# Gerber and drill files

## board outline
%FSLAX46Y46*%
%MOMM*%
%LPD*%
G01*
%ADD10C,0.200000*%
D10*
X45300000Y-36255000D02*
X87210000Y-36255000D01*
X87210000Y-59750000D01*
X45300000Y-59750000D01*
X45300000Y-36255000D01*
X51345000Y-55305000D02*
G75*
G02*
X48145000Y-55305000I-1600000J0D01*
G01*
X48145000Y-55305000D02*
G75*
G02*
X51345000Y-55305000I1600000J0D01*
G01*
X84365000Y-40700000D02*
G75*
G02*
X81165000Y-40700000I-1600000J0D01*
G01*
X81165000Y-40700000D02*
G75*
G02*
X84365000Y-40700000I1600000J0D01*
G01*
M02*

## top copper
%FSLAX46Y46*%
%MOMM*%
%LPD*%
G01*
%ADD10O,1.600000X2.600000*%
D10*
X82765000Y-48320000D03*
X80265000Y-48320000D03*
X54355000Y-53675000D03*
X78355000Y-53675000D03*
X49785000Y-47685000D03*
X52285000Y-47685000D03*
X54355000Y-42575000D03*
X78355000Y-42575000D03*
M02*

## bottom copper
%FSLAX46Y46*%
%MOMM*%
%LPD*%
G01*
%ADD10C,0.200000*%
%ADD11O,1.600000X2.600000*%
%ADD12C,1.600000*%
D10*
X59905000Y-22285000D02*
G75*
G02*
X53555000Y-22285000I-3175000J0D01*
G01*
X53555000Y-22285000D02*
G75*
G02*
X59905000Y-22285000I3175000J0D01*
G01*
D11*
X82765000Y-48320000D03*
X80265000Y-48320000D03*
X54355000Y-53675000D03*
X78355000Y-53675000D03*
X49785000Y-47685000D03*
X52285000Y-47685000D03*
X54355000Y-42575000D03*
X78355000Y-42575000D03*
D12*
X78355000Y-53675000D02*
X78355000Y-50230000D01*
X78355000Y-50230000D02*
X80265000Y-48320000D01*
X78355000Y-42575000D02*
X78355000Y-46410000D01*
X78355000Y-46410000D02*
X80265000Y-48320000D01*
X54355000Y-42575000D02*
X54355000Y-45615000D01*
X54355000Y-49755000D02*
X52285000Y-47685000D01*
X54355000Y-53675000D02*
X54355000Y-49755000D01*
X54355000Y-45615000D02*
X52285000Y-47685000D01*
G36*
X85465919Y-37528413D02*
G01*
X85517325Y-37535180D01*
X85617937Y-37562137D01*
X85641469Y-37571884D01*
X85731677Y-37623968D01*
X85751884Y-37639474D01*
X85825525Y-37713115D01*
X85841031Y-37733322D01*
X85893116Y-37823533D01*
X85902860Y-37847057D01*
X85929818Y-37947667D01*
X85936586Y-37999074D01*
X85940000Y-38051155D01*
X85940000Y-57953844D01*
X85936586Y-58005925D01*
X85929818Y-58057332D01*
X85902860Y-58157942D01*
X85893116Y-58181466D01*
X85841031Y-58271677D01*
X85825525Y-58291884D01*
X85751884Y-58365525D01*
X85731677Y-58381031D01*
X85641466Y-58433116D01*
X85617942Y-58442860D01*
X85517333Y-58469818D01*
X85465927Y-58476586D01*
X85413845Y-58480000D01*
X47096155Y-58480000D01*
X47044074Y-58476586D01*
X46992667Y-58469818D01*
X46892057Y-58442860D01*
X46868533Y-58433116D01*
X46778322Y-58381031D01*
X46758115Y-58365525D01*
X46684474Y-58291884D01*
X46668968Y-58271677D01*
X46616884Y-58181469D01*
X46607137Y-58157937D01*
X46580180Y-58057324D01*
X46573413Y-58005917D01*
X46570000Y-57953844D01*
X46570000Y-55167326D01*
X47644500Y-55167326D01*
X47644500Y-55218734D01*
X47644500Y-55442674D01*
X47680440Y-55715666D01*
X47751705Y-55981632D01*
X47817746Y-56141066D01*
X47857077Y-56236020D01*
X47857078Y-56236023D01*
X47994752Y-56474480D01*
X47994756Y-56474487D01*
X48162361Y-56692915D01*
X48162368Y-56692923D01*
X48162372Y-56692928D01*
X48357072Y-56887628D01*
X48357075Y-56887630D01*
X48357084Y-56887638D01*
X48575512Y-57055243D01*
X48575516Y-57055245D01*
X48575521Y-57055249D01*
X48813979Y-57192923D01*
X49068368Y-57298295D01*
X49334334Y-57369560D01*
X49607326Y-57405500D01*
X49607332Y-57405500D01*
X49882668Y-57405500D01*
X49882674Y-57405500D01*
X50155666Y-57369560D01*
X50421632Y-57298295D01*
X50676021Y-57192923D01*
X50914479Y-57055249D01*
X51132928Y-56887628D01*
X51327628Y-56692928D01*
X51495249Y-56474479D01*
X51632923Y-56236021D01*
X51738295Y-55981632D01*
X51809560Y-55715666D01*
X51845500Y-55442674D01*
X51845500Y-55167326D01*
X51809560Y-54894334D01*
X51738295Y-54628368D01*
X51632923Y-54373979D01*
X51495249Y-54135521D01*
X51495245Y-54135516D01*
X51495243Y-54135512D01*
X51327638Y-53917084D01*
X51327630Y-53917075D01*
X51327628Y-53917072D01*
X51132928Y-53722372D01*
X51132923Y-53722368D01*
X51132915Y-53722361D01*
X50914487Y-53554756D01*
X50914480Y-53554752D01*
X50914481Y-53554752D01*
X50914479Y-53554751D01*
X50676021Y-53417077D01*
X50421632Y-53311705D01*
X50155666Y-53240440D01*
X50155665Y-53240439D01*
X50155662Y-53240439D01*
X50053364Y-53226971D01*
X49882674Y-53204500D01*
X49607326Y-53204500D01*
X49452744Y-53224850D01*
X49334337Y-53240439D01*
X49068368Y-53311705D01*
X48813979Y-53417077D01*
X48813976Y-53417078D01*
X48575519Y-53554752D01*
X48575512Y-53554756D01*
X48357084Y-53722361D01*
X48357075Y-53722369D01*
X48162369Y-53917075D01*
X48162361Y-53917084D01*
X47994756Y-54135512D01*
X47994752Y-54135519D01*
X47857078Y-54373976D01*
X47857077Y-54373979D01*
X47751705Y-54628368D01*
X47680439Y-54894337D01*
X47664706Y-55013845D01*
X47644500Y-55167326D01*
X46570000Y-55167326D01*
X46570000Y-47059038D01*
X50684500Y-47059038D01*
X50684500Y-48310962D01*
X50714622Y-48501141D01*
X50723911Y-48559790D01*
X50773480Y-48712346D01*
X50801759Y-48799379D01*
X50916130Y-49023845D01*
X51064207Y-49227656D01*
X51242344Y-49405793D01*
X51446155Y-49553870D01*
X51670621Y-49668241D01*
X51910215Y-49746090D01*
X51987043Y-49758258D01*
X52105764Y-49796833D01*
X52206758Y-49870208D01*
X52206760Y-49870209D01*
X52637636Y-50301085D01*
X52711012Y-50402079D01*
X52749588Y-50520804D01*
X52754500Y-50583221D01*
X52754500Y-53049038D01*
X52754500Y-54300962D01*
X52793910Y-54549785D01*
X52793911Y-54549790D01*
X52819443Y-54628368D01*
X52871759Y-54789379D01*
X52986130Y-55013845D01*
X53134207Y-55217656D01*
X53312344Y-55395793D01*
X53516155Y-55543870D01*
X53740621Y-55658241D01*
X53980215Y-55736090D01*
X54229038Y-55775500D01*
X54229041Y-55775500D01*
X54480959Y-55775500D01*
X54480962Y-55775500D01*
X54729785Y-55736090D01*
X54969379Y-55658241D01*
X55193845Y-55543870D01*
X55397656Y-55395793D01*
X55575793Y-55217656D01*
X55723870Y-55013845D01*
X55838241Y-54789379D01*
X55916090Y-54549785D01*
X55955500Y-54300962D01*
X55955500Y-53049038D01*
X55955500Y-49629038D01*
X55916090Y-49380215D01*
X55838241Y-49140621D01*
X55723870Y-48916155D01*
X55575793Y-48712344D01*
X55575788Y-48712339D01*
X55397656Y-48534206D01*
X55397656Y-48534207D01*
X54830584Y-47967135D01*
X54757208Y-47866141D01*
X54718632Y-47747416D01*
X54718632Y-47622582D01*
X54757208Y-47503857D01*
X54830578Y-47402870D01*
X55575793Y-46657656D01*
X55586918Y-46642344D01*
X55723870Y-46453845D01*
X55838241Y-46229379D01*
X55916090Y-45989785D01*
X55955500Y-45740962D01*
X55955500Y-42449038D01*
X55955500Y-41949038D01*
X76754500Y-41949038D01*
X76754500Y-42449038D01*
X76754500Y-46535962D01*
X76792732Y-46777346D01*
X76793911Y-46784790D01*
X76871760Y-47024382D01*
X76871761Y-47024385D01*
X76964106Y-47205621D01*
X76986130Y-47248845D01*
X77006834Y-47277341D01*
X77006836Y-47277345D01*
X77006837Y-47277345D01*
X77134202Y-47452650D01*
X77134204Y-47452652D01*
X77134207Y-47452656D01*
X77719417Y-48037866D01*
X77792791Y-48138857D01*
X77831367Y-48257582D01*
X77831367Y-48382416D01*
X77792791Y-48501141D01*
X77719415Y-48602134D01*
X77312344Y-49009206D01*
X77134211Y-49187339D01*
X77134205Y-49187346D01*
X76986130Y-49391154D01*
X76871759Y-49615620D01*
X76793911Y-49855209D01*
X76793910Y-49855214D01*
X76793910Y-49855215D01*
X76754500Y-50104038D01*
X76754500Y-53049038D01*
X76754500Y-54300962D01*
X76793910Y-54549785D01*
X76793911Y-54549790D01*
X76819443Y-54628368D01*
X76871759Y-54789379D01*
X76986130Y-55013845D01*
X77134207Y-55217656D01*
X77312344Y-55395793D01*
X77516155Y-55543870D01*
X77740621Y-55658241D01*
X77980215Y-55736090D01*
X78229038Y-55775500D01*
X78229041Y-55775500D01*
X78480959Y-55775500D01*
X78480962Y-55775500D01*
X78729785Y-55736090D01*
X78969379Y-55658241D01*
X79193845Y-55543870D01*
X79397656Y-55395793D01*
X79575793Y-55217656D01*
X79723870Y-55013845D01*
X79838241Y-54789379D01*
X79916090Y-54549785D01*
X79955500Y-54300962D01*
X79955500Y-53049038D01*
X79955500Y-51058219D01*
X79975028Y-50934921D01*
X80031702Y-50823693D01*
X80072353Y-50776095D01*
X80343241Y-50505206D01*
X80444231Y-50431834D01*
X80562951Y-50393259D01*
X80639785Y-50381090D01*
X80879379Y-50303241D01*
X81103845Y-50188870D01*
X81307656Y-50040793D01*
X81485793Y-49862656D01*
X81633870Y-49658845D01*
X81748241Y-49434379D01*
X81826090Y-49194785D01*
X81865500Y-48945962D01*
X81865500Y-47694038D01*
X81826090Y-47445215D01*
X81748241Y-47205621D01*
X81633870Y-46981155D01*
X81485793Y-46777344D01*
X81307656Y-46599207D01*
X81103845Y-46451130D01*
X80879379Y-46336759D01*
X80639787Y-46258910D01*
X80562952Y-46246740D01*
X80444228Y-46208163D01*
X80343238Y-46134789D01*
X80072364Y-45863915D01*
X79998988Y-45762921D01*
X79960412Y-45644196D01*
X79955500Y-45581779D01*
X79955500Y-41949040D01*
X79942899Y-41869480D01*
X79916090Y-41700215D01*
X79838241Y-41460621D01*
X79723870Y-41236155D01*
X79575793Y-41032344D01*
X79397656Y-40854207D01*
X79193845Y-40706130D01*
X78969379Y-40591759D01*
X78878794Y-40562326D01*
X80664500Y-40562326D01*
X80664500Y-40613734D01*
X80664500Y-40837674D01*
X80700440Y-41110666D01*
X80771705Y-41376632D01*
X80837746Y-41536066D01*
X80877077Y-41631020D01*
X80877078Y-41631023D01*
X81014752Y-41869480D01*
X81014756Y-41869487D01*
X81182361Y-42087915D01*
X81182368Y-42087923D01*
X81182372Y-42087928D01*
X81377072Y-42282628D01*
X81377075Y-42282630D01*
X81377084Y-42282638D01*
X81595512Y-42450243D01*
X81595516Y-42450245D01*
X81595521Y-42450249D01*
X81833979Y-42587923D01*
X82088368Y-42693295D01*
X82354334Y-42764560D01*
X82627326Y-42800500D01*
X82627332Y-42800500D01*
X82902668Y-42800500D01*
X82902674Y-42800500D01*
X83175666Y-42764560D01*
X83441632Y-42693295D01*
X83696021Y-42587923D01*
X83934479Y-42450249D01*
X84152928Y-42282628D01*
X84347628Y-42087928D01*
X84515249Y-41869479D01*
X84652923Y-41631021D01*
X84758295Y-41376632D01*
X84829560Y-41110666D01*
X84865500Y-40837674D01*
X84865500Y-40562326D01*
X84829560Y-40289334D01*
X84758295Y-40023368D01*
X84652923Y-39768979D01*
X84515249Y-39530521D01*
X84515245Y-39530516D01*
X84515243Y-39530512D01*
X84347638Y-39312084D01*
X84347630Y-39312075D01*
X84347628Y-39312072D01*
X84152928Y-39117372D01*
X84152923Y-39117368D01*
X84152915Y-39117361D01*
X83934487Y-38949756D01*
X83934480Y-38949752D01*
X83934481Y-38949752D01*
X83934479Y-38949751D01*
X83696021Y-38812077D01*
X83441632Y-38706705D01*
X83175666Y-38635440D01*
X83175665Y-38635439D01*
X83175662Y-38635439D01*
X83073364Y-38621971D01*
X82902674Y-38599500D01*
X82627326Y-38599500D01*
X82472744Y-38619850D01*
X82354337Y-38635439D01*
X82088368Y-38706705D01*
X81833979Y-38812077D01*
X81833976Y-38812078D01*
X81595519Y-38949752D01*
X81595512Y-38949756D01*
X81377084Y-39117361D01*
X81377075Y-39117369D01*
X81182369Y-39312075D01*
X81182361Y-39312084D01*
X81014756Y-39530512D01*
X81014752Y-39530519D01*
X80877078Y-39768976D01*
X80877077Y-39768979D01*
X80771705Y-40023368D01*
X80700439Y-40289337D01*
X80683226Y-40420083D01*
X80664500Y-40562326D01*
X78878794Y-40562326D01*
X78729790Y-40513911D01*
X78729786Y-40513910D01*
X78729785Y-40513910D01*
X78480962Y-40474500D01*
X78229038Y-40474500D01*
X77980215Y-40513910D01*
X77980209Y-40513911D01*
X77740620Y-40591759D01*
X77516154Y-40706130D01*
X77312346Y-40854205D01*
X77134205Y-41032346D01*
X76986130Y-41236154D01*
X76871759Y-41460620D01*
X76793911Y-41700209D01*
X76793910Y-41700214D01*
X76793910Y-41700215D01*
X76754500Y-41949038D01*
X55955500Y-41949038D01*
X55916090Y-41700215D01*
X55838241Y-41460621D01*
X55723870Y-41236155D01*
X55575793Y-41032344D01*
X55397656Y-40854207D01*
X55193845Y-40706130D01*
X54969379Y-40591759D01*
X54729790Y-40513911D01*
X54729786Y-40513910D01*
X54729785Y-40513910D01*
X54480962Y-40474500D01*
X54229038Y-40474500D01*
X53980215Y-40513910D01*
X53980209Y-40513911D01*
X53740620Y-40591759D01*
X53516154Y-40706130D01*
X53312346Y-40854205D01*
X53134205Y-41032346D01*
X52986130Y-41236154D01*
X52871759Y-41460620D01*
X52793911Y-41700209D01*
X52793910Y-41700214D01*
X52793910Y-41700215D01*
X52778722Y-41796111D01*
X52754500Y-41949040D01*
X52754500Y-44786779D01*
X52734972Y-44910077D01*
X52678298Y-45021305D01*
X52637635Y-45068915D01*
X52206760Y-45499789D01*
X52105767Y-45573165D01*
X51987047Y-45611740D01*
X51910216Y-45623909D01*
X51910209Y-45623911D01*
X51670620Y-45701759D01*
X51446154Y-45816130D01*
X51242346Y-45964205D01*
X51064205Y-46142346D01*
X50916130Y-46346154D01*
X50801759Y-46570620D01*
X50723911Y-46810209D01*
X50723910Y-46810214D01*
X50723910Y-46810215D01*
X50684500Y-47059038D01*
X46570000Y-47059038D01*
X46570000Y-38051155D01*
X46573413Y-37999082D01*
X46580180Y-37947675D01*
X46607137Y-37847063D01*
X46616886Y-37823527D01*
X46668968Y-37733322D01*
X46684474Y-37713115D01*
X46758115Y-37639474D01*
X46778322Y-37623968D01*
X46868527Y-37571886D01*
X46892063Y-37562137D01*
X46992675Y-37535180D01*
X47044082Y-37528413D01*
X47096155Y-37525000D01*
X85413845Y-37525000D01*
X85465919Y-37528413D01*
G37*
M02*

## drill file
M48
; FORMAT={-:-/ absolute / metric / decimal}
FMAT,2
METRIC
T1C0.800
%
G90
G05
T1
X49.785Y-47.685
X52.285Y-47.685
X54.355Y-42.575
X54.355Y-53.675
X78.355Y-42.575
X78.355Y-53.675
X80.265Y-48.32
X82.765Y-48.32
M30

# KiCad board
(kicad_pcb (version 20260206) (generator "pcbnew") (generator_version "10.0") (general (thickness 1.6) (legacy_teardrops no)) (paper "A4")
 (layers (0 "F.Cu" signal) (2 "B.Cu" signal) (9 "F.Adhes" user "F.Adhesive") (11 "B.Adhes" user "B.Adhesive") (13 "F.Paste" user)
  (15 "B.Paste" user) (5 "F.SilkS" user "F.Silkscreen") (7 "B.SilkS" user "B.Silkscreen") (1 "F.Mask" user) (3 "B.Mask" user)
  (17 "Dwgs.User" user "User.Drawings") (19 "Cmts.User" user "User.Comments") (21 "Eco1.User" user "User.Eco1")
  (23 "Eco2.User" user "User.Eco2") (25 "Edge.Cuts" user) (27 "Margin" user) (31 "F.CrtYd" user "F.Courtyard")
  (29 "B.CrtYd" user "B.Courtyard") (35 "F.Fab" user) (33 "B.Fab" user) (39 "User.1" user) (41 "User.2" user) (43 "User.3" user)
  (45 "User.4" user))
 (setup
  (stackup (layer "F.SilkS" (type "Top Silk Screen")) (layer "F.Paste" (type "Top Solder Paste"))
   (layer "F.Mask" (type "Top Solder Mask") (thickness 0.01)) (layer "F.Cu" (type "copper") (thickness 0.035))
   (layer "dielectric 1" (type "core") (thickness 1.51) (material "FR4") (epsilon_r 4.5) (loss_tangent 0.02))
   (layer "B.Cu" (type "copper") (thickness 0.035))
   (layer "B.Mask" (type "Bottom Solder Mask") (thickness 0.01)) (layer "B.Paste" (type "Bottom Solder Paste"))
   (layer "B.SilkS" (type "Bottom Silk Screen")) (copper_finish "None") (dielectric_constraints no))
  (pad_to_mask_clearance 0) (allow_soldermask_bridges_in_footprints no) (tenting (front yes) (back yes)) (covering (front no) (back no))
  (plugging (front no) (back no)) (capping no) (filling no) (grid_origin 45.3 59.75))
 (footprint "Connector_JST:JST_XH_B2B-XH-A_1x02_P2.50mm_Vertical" (layer "F.Cu") (at 82.765 48.32 180)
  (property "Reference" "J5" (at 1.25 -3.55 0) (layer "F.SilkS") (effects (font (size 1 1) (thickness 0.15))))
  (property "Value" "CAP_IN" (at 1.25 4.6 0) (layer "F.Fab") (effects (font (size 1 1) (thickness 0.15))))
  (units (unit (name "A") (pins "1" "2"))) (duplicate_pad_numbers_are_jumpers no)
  (pad "1" thru_hole oval (at 0 0 180) (size 1.6 2.6) (drill 0.8) (layers "*.Cu" "*.Mask") (remove_unused_layers no) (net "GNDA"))
  (pad "2" thru_hole oval (at 2.5 0 180) (size 1.6 2.6) (drill 0.8) (layers "*.Cu" "*.Mask") (remove_unused_layers no) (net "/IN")))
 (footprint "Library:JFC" (layer "F.Cu") (at 54.355 53.675)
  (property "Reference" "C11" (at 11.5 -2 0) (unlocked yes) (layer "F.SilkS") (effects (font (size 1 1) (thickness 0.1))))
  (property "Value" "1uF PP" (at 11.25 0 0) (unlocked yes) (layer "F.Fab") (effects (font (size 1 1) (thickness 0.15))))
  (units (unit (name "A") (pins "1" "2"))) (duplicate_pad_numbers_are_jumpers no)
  (pad "1" thru_hole oval (at 0 0) (size 1.6 2.6) (drill 0.8) (layers "*.Cu" "*.Mask") (remove_unused_layers no) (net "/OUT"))
  (pad "2" thru_hole oval (at 24 0) (size 1.6 2.6) (drill 0.8) (layers "*.Cu" "*.Mask") (remove_unused_layers no) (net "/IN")))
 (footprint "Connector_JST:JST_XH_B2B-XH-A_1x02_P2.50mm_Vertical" (layer "F.Cu") (at 49.785 47.685)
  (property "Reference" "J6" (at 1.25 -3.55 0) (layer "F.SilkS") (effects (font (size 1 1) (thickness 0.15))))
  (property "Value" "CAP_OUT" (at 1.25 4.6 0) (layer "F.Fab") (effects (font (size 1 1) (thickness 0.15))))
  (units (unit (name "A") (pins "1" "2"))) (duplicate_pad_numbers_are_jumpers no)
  (pad "1" thru_hole oval (at 0 0) (size 1.6 2.6) (drill 0.8) (layers "*.Cu" "*.Mask") (remove_unused_layers no) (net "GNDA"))
  (pad "2" thru_hole oval (at 2.5 0) (size 1.6 2.6) (drill 0.8) (layers "*.Cu" "*.Mask") (remove_unused_layers no) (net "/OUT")))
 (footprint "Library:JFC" (layer "F.Cu") (at 54.355 42.575)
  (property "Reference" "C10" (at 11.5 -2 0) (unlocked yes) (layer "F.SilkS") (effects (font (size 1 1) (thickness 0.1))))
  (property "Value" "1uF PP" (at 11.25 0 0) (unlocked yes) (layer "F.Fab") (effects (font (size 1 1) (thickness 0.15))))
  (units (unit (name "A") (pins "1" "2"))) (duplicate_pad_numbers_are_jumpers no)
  (pad "1" thru_hole oval (at 0 0) (size 1.6 2.6) (drill 0.8) (layers "*.Cu" "*.Mask") (remove_unused_layers no) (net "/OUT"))
  (pad "2" thru_hole oval (at 24 0) (size 1.6 2.6) (drill 0.8) (layers "*.Cu" "*.Mask") (remove_unused_layers no) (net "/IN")))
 (gr_circle (center 56.73 22.285) (end 59.905 22.285) (stroke (width 0.2) (type default)) (fill no) (layer "B.Cu"))
 (gr_rect (start 45.3 36.255) (end 87.21 59.75) (stroke (width 0.2) (type solid)) (fill no) (layer "Edge.Cuts"))
 (gr_circle (center 49.745 55.305) (end 51.345 55.305) (stroke (width 0.2) (type solid)) (fill no) (layer "Edge.Cuts"))
 (gr_circle (center 82.765 40.7) (end 84.365 40.7) (stroke (width 0.2) (type solid)) (fill no) (layer "Edge.Cuts"))
 (segment (start 78.355 53.675) (end 78.355 50.23) (width 1.6) (layer "B.Cu") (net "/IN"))
 (segment (start 78.355 50.23) (end 80.265 48.32) (width 1.6) (layer "B.Cu") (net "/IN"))
 (segment (start 78.355 42.575) (end 78.355 46.41) (width 1.6) (layer "B.Cu") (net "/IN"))
 (segment (start 78.355 46.41) (end 80.265 48.32) (width 1.6) (layer "B.Cu") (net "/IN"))
 (segment (start 54.355 42.575) (end 54.355 45.615) (width 1.6) (layer "B.Cu") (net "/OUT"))
 (segment (start 54.355 49.755) (end 52.285 47.685) (width 1.6) (layer "B.Cu") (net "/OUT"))
 (segment (start 54.355 53.675) (end 54.355 49.755) (width 1.6) (layer "B.Cu") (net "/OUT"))
 (segment (start 54.355 45.615) (end 52.285 47.685) (width 1.6) (layer "B.Cu") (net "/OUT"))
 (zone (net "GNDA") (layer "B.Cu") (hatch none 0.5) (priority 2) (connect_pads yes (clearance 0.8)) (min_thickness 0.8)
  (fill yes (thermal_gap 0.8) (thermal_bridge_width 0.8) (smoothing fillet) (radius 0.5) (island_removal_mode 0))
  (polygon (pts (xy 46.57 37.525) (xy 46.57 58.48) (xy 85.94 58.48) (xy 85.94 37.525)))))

